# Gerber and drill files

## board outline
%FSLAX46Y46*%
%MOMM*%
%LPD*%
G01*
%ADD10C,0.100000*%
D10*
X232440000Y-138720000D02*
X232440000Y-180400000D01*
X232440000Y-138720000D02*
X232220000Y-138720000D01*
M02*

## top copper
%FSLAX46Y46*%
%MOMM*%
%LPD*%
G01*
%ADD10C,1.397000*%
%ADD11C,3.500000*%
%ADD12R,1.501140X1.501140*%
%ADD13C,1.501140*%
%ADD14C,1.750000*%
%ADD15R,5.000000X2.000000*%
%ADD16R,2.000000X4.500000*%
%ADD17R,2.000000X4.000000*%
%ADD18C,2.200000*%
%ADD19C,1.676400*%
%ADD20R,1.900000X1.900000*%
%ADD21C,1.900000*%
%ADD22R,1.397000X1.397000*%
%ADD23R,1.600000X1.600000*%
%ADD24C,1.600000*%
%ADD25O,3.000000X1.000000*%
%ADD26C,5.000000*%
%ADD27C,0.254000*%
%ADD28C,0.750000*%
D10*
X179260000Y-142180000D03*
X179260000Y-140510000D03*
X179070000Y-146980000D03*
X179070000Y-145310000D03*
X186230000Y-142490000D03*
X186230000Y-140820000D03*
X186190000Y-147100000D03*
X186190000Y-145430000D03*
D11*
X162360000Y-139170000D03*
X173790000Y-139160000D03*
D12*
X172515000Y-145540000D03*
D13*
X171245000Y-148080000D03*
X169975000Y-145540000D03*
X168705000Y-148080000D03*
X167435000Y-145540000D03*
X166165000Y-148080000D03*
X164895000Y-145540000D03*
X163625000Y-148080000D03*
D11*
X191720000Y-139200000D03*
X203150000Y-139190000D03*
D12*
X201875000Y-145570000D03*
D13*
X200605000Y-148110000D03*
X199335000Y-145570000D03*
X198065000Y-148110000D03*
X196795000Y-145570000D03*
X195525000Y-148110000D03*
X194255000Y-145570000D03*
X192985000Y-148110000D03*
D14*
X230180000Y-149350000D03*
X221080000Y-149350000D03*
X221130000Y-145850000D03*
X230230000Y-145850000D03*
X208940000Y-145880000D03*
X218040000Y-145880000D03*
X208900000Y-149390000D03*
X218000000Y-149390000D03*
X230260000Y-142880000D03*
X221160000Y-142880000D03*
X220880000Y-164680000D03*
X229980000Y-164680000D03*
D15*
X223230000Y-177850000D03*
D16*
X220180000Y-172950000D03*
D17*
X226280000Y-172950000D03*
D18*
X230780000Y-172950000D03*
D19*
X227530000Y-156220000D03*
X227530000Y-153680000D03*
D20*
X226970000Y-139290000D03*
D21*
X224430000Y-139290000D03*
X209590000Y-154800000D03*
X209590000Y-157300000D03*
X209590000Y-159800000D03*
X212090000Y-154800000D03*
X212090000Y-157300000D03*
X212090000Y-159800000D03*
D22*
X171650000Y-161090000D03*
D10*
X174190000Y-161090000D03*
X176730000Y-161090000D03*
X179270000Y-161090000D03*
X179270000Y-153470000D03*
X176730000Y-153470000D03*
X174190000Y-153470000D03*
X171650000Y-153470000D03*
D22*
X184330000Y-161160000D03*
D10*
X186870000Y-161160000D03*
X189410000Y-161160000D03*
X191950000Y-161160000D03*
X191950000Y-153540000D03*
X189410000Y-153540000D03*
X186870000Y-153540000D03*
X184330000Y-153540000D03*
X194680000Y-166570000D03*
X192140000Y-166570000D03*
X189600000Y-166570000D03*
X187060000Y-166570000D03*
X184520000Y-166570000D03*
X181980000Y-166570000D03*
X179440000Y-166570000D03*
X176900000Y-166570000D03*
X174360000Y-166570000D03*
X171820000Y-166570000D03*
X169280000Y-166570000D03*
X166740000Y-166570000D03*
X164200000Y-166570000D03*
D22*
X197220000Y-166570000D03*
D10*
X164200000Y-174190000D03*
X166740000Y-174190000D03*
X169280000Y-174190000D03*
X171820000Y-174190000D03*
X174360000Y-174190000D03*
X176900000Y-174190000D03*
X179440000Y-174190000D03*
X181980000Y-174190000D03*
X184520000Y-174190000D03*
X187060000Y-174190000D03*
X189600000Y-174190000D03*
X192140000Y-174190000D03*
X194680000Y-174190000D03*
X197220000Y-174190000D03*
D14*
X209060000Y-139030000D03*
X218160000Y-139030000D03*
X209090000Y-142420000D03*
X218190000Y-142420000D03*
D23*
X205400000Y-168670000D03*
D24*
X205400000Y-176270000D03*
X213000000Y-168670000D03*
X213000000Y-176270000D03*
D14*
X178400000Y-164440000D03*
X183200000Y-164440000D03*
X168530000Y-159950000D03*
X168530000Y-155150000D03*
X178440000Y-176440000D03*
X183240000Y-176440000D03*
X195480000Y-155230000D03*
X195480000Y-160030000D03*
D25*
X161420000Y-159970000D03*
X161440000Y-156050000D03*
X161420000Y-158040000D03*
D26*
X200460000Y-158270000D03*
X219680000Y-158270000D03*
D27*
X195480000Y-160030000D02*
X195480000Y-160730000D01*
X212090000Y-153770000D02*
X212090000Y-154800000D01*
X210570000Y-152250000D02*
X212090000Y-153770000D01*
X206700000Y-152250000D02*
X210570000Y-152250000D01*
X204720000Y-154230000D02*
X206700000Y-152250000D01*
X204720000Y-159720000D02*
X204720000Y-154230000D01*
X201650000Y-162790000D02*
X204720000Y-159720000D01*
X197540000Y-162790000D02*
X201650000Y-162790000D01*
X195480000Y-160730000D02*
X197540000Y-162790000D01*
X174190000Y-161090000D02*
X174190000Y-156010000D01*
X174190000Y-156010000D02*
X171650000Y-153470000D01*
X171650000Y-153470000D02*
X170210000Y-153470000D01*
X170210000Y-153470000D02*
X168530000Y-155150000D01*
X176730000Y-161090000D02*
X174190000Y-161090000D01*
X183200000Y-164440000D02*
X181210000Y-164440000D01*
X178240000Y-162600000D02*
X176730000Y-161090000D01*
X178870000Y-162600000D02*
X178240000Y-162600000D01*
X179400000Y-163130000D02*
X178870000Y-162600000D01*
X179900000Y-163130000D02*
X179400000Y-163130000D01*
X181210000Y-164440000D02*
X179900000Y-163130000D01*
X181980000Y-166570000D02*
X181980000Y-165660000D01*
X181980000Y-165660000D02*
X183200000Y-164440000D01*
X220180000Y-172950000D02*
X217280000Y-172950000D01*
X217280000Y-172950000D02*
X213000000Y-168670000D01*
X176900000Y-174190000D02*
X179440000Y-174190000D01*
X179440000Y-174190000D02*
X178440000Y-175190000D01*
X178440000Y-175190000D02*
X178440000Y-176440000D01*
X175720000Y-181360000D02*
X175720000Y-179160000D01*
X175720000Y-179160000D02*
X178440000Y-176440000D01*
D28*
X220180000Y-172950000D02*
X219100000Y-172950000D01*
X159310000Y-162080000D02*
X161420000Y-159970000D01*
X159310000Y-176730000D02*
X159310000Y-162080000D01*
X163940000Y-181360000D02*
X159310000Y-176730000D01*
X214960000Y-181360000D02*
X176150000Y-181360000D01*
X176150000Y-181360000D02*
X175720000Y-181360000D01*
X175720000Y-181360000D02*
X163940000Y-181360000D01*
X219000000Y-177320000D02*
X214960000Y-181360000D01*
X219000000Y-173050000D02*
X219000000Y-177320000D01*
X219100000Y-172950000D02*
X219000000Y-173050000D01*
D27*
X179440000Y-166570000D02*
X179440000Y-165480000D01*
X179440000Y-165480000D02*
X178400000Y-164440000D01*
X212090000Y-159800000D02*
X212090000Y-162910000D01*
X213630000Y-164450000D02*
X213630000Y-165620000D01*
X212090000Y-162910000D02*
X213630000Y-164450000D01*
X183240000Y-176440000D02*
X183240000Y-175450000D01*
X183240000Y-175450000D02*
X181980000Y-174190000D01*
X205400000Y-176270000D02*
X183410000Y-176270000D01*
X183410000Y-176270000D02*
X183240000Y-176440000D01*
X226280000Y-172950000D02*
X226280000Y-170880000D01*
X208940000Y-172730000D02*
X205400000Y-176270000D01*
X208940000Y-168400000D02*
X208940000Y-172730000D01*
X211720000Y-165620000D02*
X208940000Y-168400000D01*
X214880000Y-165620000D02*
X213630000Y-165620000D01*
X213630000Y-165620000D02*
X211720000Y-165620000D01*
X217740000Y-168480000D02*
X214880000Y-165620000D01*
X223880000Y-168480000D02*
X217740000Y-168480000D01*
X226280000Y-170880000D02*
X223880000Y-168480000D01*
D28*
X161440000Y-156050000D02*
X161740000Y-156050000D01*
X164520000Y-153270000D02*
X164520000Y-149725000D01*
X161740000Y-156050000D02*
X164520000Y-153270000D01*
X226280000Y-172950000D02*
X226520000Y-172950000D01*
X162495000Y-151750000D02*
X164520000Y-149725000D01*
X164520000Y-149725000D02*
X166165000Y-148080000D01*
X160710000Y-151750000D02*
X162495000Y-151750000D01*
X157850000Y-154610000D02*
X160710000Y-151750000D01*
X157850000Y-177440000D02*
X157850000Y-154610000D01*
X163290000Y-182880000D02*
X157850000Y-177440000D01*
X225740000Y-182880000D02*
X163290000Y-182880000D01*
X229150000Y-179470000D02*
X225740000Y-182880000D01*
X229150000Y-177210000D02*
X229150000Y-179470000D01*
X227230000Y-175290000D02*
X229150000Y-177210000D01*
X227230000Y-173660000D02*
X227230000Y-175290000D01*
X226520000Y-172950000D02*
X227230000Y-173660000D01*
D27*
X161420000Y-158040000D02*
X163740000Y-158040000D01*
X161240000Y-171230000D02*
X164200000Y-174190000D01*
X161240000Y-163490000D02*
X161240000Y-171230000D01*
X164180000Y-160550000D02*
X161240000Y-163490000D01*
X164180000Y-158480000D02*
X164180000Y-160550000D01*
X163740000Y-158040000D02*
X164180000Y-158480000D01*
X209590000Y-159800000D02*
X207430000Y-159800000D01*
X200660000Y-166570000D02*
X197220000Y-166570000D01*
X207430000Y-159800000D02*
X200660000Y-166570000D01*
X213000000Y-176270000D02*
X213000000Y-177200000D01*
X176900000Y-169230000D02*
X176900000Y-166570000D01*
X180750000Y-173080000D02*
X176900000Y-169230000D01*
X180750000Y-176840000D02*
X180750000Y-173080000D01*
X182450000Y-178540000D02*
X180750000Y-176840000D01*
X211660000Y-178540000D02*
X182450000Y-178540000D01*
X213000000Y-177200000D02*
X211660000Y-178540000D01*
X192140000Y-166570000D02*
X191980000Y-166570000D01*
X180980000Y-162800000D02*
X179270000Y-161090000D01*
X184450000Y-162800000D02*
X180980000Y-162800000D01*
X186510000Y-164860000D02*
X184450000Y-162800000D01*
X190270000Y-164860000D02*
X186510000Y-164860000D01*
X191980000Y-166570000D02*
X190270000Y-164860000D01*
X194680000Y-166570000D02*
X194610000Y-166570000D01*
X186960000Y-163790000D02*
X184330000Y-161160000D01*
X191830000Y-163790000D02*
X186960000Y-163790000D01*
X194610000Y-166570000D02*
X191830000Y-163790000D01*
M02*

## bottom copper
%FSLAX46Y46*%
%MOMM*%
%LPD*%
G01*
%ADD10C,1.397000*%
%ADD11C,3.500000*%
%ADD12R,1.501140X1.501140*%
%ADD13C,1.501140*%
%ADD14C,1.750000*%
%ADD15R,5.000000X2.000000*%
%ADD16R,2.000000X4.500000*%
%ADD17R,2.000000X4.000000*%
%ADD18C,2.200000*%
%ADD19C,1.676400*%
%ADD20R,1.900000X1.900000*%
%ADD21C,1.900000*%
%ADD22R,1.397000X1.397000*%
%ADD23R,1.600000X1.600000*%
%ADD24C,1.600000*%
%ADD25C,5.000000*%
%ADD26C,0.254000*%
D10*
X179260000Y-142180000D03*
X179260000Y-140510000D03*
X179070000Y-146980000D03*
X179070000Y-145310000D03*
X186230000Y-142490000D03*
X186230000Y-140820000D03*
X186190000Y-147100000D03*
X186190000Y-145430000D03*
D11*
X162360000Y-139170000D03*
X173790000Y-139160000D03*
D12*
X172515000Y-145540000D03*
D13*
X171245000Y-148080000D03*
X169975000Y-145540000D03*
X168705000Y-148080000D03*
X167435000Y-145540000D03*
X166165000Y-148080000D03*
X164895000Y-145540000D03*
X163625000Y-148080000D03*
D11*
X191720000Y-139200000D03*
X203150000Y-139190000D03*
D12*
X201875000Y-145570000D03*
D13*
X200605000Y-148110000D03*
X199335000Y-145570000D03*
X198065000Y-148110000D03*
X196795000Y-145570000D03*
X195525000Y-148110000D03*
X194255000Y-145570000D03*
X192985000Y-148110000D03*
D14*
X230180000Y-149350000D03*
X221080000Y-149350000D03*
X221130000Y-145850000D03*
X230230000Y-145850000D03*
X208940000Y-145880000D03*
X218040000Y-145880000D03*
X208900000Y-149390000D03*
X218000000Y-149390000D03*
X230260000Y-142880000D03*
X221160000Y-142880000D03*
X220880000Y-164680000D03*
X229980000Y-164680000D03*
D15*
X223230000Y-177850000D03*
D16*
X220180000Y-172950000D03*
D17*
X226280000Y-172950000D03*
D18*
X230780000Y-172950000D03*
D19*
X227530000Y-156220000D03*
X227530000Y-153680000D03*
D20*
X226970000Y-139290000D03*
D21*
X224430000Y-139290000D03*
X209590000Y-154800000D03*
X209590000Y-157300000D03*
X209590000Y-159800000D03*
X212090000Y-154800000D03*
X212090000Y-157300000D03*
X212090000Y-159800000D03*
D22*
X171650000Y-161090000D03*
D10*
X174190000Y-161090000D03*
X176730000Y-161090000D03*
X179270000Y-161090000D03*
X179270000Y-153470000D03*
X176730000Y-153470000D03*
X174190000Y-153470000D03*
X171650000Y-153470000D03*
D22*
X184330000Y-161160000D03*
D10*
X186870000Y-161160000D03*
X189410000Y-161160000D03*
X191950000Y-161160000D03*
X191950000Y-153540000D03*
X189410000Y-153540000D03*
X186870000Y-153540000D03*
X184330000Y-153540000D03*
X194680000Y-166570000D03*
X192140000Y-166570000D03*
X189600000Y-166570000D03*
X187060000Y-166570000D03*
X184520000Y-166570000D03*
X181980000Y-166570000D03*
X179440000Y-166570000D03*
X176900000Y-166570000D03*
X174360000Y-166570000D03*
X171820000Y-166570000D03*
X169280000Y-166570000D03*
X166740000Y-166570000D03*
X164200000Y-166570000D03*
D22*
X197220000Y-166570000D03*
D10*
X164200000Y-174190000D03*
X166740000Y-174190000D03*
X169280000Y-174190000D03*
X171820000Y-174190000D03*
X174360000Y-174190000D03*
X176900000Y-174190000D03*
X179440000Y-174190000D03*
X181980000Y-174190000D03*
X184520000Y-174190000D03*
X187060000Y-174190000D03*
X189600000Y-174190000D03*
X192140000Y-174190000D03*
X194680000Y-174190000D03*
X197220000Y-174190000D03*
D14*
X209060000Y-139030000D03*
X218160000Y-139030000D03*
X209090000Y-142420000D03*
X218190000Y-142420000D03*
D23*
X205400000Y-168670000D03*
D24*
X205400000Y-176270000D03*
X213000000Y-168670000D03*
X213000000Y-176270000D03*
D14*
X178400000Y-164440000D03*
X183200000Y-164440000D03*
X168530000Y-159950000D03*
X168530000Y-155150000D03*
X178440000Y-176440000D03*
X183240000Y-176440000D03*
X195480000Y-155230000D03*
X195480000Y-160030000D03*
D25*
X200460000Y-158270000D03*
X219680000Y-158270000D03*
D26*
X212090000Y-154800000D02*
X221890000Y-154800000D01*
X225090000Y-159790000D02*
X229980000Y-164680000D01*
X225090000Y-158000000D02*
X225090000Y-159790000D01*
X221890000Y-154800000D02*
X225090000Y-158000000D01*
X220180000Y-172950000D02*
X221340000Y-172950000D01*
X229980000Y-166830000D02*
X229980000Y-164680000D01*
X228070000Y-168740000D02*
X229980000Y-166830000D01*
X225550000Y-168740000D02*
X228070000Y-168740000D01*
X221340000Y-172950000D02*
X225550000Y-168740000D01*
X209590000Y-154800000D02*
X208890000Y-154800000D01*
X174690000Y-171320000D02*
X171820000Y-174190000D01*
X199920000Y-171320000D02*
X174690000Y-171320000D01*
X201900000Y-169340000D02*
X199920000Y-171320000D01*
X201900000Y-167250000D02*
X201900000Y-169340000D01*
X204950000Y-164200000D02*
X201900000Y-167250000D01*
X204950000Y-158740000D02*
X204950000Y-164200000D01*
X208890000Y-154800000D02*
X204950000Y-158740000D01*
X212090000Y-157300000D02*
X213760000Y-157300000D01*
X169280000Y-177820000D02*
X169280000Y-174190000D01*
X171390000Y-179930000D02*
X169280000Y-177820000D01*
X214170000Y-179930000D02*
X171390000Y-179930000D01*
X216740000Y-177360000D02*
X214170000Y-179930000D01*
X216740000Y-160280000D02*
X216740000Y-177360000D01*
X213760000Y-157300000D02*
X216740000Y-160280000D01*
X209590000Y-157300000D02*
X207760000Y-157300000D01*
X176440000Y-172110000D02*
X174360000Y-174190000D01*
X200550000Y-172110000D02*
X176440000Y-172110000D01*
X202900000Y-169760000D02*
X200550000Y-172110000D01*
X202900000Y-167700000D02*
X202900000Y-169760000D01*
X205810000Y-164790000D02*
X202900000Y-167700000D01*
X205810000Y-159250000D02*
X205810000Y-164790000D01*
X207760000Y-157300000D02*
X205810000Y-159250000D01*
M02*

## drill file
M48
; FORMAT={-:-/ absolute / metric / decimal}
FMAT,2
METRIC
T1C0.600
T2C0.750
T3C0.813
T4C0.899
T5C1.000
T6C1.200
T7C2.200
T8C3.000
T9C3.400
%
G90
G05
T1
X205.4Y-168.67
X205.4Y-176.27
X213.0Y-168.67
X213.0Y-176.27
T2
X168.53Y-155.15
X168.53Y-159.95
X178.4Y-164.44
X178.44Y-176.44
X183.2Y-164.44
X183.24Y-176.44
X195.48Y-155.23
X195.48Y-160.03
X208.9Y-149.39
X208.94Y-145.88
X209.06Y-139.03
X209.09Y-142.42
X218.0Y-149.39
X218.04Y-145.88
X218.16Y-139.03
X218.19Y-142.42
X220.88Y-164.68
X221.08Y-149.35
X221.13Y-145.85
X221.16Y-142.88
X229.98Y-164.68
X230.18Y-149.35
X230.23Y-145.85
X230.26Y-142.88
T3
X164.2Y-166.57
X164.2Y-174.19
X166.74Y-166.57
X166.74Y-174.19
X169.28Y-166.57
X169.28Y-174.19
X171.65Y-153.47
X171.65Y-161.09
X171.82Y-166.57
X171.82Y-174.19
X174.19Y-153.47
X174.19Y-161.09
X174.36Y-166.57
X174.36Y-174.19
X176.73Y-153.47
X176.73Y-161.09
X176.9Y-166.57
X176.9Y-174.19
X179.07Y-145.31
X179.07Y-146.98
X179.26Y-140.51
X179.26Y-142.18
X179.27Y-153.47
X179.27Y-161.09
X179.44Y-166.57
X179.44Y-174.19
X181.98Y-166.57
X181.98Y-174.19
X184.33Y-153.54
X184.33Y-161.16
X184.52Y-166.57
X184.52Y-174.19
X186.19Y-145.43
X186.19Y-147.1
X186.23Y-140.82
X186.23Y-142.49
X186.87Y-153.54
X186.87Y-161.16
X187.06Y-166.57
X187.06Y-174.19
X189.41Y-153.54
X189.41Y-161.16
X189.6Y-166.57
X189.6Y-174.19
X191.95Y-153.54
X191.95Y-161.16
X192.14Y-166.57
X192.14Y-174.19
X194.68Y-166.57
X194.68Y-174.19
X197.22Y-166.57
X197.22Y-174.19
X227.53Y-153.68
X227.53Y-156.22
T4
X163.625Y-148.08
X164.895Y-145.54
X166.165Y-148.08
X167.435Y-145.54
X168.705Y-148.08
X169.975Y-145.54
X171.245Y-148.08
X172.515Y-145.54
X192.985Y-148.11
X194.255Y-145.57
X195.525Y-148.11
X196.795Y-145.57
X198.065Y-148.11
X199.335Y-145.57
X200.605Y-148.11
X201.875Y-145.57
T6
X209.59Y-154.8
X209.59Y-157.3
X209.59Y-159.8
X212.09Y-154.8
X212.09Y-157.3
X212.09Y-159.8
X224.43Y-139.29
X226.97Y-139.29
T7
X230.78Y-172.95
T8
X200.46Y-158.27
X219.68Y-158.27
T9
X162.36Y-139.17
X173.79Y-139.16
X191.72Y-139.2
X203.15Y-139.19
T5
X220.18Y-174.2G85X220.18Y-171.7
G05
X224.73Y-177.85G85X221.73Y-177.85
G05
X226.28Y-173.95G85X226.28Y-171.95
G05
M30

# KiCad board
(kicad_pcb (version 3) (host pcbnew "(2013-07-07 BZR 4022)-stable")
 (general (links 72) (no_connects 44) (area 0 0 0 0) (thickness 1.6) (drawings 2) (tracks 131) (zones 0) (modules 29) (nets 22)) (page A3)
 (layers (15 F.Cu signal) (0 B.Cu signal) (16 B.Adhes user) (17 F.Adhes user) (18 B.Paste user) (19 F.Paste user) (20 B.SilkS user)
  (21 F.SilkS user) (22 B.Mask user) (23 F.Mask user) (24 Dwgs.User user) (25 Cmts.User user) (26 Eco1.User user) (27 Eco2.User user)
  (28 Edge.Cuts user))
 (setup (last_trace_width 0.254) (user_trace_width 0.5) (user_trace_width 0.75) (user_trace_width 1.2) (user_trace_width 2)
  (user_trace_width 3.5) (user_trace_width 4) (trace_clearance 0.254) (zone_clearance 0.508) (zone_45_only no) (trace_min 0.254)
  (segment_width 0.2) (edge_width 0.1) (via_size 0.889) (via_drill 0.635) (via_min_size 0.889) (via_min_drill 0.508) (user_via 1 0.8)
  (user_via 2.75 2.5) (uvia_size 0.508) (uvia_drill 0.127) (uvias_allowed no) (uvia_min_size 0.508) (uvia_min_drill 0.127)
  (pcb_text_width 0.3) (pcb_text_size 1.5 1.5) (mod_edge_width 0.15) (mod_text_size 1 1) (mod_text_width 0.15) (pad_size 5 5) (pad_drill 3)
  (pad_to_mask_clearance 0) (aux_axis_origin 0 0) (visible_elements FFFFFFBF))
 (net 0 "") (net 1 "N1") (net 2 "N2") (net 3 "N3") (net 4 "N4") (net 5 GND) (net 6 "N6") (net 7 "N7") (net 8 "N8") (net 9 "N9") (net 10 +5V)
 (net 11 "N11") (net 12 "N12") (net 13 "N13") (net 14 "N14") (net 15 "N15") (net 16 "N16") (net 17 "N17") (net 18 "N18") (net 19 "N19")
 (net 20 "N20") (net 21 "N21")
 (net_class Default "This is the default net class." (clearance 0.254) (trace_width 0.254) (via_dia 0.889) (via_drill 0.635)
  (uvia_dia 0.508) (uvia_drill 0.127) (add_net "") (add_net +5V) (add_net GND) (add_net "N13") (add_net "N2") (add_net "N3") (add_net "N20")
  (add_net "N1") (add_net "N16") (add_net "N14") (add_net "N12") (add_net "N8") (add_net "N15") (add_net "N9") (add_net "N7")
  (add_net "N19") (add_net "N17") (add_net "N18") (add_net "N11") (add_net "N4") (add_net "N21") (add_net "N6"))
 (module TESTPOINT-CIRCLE (layer F.Cu) (at 179.26 141.35 90)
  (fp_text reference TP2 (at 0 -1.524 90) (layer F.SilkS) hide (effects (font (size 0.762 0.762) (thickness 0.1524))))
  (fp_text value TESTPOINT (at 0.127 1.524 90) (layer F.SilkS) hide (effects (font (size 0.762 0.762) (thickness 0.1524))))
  (pad 1 thru_hole circle (at -0.83 0 90) (size 1.397 1.397) (drill 0.8128) (layers *.Cu *.Mask F.SilkS) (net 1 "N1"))
  (pad 1 thru_hole circle (at 0.84 0 90) (size 1.397 1.397) (drill 0.8128) (layers *.Cu *.Mask F.SilkS) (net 1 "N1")))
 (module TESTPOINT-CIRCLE (layer F.Cu) (at 179.07 146.15 90)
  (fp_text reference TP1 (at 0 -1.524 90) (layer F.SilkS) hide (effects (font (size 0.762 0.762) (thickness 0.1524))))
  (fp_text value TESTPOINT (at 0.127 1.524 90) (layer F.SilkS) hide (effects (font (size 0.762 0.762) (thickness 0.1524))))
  (pad 1 thru_hole circle (at -0.83 0 90) (size 1.397 1.397) (drill 0.8128) (layers *.Cu *.Mask F.SilkS) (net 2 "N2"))
  (pad 1 thru_hole circle (at 0.84 0 90) (size 1.397 1.397) (drill 0.8128) (layers *.Cu *.Mask F.SilkS) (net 2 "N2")))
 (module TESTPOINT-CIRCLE (layer F.Cu) (at 186.23 141.66 90)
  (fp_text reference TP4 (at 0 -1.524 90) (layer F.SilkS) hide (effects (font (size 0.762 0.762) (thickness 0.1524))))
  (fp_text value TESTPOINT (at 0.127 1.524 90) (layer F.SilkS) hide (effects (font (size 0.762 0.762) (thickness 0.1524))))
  (pad 1 thru_hole circle (at -0.83 0 90) (size 1.397 1.397) (drill 0.8128) (layers *.Cu *.Mask F.SilkS) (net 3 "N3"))
  (pad 1 thru_hole circle (at 0.84 0 90) (size 1.397 1.397) (drill 0.8128) (layers *.Cu *.Mask F.SilkS) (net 3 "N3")))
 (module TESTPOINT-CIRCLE (layer F.Cu) (at 186.19 146.27 90)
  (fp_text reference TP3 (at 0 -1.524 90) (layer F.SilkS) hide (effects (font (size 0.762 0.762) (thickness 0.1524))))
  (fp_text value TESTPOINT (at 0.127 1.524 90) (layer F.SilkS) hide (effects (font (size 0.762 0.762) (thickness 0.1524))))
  (pad 1 thru_hole circle (at -0.83 0 90) (size 1.397 1.397) (drill 0.8128) (layers *.Cu *.Mask F.SilkS) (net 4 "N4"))
  (pad 1 thru_hole circle (at 0.84 0 90) (size 1.397 1.397) (drill 0.8128) (layers *.Cu *.Mask F.SilkS) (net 4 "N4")))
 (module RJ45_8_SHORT (layer F.Cu) (at 168.07 139.19 180)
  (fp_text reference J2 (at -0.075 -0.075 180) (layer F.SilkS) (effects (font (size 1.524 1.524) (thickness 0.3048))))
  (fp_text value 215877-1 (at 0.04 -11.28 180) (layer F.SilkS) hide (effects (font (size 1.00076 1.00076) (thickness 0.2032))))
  (pad Hole thru_hole circle (at 5.71 0.02 180) (size 3.5 3.5) (drill 3.4) (layers *.Cu *.Mask F.SilkS))
  (pad Hole thru_hole circle (at -5.72 0.03 180) (size 3.5 3.5) (drill 3.4) (layers *.Cu *.Mask F.SilkS))
  (pad 1 thru_hole rect (at -4.445 -6.35 180) (size 1.50114 1.50114) (drill 0.89916) (layers *.Cu *.Mask F.SilkS) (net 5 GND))
  (pad 2 thru_hole circle (at -3.175 -8.89 180) (size 1.50114 1.50114) (drill 0.89916) (layers *.Cu *.Mask F.SilkS) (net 5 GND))
  (pad 3 thru_hole circle (at -1.905 -6.35 180) (size 1.50114 1.50114) (drill 0.89916) (layers *.Cu *.Mask F.SilkS) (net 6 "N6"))
  (pad 4 thru_hole circle (at -0.635 -8.89 180) (size 1.50114 1.50114) (drill 0.89916) (layers *.Cu *.Mask F.SilkS) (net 1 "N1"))
  (pad 5 thru_hole circle (at 0.635 -6.35 180) (size 1.50114 1.50114) (drill 0.89916) (layers *.Cu *.Mask F.SilkS) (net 2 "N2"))
  (pad 6 thru_hole circle (at 1.905 -8.89 180) (size 1.50114 1.50114) (drill 0.89916) (layers *.Cu *.Mask F.SilkS) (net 5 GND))
  (pad 7 thru_hole circle (at 3.175 -6.35 180) (size 1.50114 1.50114) (drill 0.89916) (layers *.Cu *.Mask F.SilkS) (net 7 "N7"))
  (pad 8 thru_hole circle (at 4.445 -8.89 180) (size 1.50114 1.50114) (drill 0.89916) (layers *.Cu *.Mask F.SilkS) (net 7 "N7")))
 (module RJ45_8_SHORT (layer F.Cu) (at 197.43 139.22 180)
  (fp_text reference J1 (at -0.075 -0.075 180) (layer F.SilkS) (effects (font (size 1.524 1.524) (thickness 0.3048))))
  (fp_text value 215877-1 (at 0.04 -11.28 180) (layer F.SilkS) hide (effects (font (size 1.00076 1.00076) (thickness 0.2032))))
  (pad Hole thru_hole circle (at 5.71 0.02 180) (size 3.5 3.5) (drill 3.4) (layers *.Cu *.Mask F.SilkS))
  (pad Hole thru_hole circle (at -5.72 0.03 180) (size 3.5 3.5) (drill 3.4) (layers *.Cu *.Mask F.SilkS))
  (pad 1 thru_hole rect (at -4.445 -6.35 180) (size 1.50114 1.50114) (drill 0.89916) (layers *.Cu *.Mask F.SilkS) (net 5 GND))
  (pad 2 thru_hole circle (at -3.175 -8.89 180) (size 1.50114 1.50114) (drill 0.89916) (layers *.Cu *.Mask F.SilkS) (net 5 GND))
  (pad 3 thru_hole circle (at -1.905 -6.35 180) (size 1.50114 1.50114) (drill 0.89916) (layers *.Cu *.Mask F.SilkS) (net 6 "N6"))
  (pad 4 thru_hole circle (at -0.635 -8.89 180) (size 1.50114 1.50114) (drill 0.89916) (layers *.Cu *.Mask F.SilkS) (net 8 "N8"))
  (pad 5 thru_hole circle (at 0.635 -6.35 180) (size 1.50114 1.50114) (drill 0.89916) (layers *.Cu *.Mask F.SilkS) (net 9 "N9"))
  (pad 6 thru_hole circle (at 1.905 -8.89 180) (size 1.50114 1.50114) (drill 0.89916) (layers *.Cu *.Mask F.SilkS) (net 5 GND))
  (pad 7 thru_hole circle (at 3.175 -6.35 180) (size 1.50114 1.50114) (drill 0.89916) (layers *.Cu *.Mask F.SilkS) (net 7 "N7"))
  (pad 8 thru_hole circle (at 4.445 -8.89 180) (size 1.50114 1.50114) (drill 0.89916) (layers *.Cu *.Mask F.SilkS) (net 7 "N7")))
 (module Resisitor (layer F.Cu) (at 225.58 149.35 180)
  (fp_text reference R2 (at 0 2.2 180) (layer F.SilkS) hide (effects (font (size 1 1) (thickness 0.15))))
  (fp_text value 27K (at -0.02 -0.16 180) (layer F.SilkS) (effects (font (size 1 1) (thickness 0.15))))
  (pad 1 thru_hole circle (at -4.6 0 180) (size 1.75 1.75) (drill 0.75) (layers *.Cu *.Mask F.SilkS) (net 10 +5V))
  (pad 2 thru_hole circle (at 4.5 0 180) (size 1.75 1.75) (drill 0.75) (layers *.Cu *.Mask F.SilkS) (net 4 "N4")))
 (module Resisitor (layer F.Cu) (at 225.73 145.85)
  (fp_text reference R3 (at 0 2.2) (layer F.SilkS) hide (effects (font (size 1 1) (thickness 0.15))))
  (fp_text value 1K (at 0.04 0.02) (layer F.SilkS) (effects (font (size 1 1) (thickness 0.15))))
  (pad 1 thru_hole circle (at -4.6 0) (size 1.75 1.75) (drill 0.75) (layers *.Cu *.Mask F.SilkS) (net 4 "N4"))
  (pad 2 thru_hole circle (at 4.5 0) (size 1.75 1.75) (drill 0.75) (layers *.Cu *.Mask F.SilkS) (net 9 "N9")))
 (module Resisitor (layer F.Cu) (at 213.54 145.88)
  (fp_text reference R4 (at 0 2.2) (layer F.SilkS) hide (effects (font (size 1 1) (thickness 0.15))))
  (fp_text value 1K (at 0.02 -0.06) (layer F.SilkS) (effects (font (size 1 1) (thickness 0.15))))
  (pad 1 thru_hole circle (at -4.6 0) (size 1.75 1.75) (drill 0.75) (layers *.Cu *.Mask F.SilkS) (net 8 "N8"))
  (pad 2 thru_hole circle (at 4.5 0) (size 1.75 1.75) (drill 0.75) (layers *.Cu *.Mask F.SilkS) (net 3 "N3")))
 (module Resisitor (layer F.Cu) (at 213.5 149.39)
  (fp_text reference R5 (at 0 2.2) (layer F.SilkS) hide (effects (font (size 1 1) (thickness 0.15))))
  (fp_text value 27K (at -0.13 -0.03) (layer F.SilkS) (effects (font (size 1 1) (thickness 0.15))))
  (pad 1 thru_hole circle (at -4.6 0) (size 1.75 1.75) (drill 0.75) (layers *.Cu *.Mask F.SilkS) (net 3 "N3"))
  (pad 2 thru_hole circle (at 4.5 0) (size 1.75 1.75) (drill 0.75) (layers *.Cu *.Mask F.SilkS) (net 5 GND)))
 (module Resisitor (layer F.Cu) (at 225.66 142.88 180)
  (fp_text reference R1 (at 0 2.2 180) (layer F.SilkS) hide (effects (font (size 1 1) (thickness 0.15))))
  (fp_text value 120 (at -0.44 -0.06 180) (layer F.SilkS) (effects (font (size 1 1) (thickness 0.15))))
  (pad 1 thru_hole circle (at -4.6 0 180) (size 1.75 1.75) (drill 0.75) (layers *.Cu *.Mask F.SilkS) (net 9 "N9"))
  (pad 2 thru_hole circle (at 4.5 0 180) (size 1.75 1.75) (drill 0.75) (layers *.Cu *.Mask F.SilkS) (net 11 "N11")))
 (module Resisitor (layer F.Cu) (at 225.48 164.68)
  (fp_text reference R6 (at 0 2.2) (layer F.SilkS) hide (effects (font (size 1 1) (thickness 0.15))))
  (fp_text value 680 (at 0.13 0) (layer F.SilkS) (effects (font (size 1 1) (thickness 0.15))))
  (pad 1 thru_hole circle (at -4.6 0) (size 1.75 1.75) (drill 0.75) (layers *.Cu *.Mask F.SilkS) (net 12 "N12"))
  (pad 2 thru_hole circle (at 4.5 0) (size 1.75 1.75) (drill 0.75) (layers *.Cu *.Mask F.SilkS) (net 10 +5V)))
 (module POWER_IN (layer F.Cu) (at 227.38 176.02 180)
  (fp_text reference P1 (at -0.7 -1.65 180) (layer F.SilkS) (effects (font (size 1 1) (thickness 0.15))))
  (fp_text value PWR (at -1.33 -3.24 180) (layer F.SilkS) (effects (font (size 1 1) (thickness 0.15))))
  (pad "" thru_hole rect (at 4.15 -1.83 180) (size 5 2) (drill oval 4 1) (layers *.Cu *.Mask F.SilkS))
  (pad 1 thru_hole rect (at 7.2 3.07 180) (size 2 4.5) (drill oval 1 3.5) (layers *.Cu *.Mask F.SilkS) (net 10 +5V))
  (pad 2 thru_hole rect (at 1.1 3.07 180) (size 2 4) (drill oval 1 3) (layers *.Cu *.Mask F.SilkS) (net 5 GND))
  (pad "" thru_hole circle (at -3.4 3.07 180) (size 2.2 2.2) (drill 2.2) (layers *.Cu *.Mask F.SilkS)))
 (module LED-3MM (layer F.Cu) (at 227.53 154.95 90)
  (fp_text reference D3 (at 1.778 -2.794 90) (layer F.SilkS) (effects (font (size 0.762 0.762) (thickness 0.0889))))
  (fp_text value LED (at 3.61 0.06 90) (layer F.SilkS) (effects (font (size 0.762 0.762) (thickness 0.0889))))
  (pad 1 thru_hole circle (at -1.27 0 90) (size 1.6764 1.6764) (drill 0.8128) (layers *.Cu *.Mask F.SilkS) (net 12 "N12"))
  (pad 2 thru_hole circle (at 1.27 0 90) (size 1.6764 1.6764) (drill 0.8128) (layers *.Cu *.Mask F.SilkS) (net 5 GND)))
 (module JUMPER (layer F.Cu) (at 225.7 139.29 180)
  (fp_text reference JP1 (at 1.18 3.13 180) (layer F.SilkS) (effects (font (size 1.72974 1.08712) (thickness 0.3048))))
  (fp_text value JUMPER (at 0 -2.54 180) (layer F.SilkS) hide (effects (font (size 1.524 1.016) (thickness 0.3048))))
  (pad 1 thru_hole rect (at -1.27 0 180) (size 1.9 1.9) (drill 1.2) (layers *.Cu *.Mask F.SilkS) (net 11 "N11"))
  (pad 2 thru_hole circle (at 1.27 0 180) (size 1.9 1.9) (drill 1.2) (layers *.Cu *.Mask F.SilkS) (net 8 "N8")))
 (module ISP (layer F.Cu) (at 210.69 157.8 90)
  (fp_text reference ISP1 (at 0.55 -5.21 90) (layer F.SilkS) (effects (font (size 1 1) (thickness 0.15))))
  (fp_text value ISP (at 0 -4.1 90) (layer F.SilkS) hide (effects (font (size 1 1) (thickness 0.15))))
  (pad 1 thru_hole circle (at 3 -1.1 90) (size 1.9 1.9) (drill 1.2) (layers *.Cu *.Mask F.SilkS) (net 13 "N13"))
  (pad 3 thru_hole circle (at 0.5 -1.1 90) (size 1.9 1.9) (drill 1.2) (layers *.Cu *.Mask F.SilkS) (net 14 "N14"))
  (pad 5 thru_hole circle (at -2 -1.1 90) (size 1.9 1.9) (drill 1.2) (layers *.Cu *.Mask F.SilkS) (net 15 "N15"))
  (pad 2 thru_hole circle (at 3 1.4 90) (size 1.9 1.9) (drill 1.2) (layers *.Cu *.Mask F.SilkS) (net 10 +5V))
  (pad 4 thru_hole circle (at 0.5 1.4 90) (size 1.9 1.9) (drill 1.2) (layers *.Cu *.Mask F.SilkS) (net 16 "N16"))
  (pad 6 thru_hole circle (at -2 1.4 90) (size 1.9 1.9) (drill 1.2) (layers *.Cu *.Mask F.SilkS) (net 5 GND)))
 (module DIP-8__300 (layer F.Cu) (at 175.46 157.28)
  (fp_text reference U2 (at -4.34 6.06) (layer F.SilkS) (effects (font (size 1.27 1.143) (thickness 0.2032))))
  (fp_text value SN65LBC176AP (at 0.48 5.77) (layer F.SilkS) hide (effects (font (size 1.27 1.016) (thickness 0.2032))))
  (pad 1 thru_hole rect (at -3.81 3.81) (size 1.397 1.397) (drill 0.8128) (layers *.Cu *.Mask F.SilkS))
  (pad 2 thru_hole circle (at -1.27 3.81) (size 1.397 1.397) (drill 0.8128) (layers *.Cu *.Mask F.SilkS) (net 10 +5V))
  (pad 3 thru_hole circle (at 1.27 3.81) (size 1.397 1.397) (drill 0.8128) (layers *.Cu *.Mask F.SilkS) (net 10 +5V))
  (pad 4 thru_hole circle (at 3.81 3.81) (size 1.397 1.397) (drill 0.8128) (layers *.Cu *.Mask F.SilkS) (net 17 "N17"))
  (pad 5 thru_hole circle (at 3.81 -3.81) (size 1.397 1.397) (drill 0.8128) (layers *.Cu *.Mask F.SilkS) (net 5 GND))
  (pad 6 thru_hole circle (at 1.27 -3.81) (size 1.397 1.397) (drill 0.8128) (layers *.Cu *.Mask F.SilkS) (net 2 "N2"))
  (pad 7 thru_hole circle (at -1.27 -3.81) (size 1.397 1.397) (drill 0.8128) (layers *.Cu *.Mask F.SilkS) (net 1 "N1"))
  (pad 8 thru_hole circle (at -3.81 -3.81) (size 1.397 1.397) (drill 0.8128) (layers *.Cu *.Mask F.SilkS) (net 10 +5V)))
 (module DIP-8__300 (layer F.Cu) (at 188.14 157.35)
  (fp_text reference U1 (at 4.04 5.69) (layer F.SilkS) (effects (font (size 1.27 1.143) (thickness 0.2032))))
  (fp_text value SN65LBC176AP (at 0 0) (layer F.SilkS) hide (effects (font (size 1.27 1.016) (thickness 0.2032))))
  (pad 1 thru_hole rect (at -3.81 3.81) (size 1.397 1.397) (drill 0.8128) (layers *.Cu *.Mask F.SilkS) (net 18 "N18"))
  (pad 2 thru_hole circle (at -1.27 3.81) (size 1.397 1.397) (drill 0.8128) (layers *.Cu *.Mask F.SilkS) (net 5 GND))
  (pad 3 thru_hole circle (at 1.27 3.81) (size 1.397 1.397) (drill 0.8128) (layers *.Cu *.Mask F.SilkS) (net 5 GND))
  (pad 4 thru_hole circle (at 3.81 3.81) (size 1.397 1.397) (drill 0.8128) (layers *.Cu *.Mask F.SilkS))
  (pad 5 thru_hole circle (at 3.81 -3.81) (size 1.397 1.397) (drill 0.8128) (layers *.Cu *.Mask F.SilkS) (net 5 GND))
  (pad 6 thru_hole circle (at 1.27 -3.81) (size 1.397 1.397) (drill 0.8128) (layers *.Cu *.Mask F.SilkS) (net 4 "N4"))
  (pad 7 thru_hole circle (at -1.27 -3.81) (size 1.397 1.397) (drill 0.8128) (layers *.Cu *.Mask F.SilkS) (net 3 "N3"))
  (pad 8 thru_hole circle (at -3.81 -3.81) (size 1.397 1.397) (drill 0.8128) (layers *.Cu *.Mask F.SilkS) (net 10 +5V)))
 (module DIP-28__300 (layer F.Cu) (at 180.71 170.38 180)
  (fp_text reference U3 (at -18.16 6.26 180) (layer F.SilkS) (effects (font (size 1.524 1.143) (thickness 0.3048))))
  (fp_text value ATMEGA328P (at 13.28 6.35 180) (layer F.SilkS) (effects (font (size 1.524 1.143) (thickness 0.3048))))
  (pad 2 thru_hole circle (at -13.97 3.81 180) (size 1.397 1.397) (drill 0.8128) (layers *.Cu *.Mask F.SilkS) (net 18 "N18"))
  (pad 3 thru_hole circle (at -11.43 3.81 180) (size 1.397 1.397) (drill 0.8128) (layers *.Cu *.Mask F.SilkS) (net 17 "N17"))
  (pad 4 thru_hole circle (at -8.89 3.81 180) (size 1.397 1.397) (drill 0.8128) (layers *.Cu *.Mask F.SilkS))
  (pad 5 thru_hole circle (at -6.35 3.81 180) (size 1.397 1.397) (drill 0.8128) (layers *.Cu *.Mask F.SilkS))
  (pad 6 thru_hole circle (at -3.81 3.81 180) (size 1.397 1.397) (drill 0.8128) (layers *.Cu *.Mask F.SilkS))
  (pad 7 thru_hole circle (at -1.27 3.81 180) (size 1.397 1.397) (drill 0.8128) (layers *.Cu *.Mask F.SilkS) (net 10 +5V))
  (pad 8 thru_hole circle (at 1.27 3.81 180) (size 1.397 1.397) (drill 0.8128) (layers *.Cu *.Mask F.SilkS) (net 5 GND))
  (pad 9 thru_hole circle (at 3.81 3.81 180) (size 1.397 1.397) (drill 0.8128) (layers *.Cu *.Mask F.SilkS) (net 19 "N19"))
  (pad 10 thru_hole circle (at 6.35 3.81 180) (size 1.397 1.397) (drill 0.8128) (layers *.Cu *.Mask F.SilkS))
  (pad 11 thru_hole circle (at 8.89 3.81 180) (size 1.397 1.397) (drill 0.8128) (layers *.Cu *.Mask F.SilkS))
  (pad 12 thru_hole circle (at 11.43 3.81 180) (size 1.397 1.397) (drill 0.8128) (layers *.Cu *.Mask F.SilkS))
  (pad 13 thru_hole circle (at 13.97 3.81 180) (size 1.397 1.397) (drill 0.8128) (layers *.Cu *.Mask F.SilkS))
  (pad 14 thru_hole circle (at 16.51 3.81 180) (size 1.397 1.397) (drill 0.8128) (layers *.Cu *.Mask F.SilkS))
  (pad 1 thru_hole rect (at -16.51 3.81 180) (size 1.397 1.397) (drill 0.8128) (layers *.Cu *.Mask F.SilkS) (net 15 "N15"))
  (pad 15 thru_hole circle (at 16.51 -3.81 180) (size 1.397 1.397) (drill 0.8128) (layers *.Cu *.Mask F.SilkS) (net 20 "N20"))
  (pad 16 thru_hole circle (at 13.97 -3.81 180) (size 1.397 1.397) (drill 0.8128) (layers *.Cu *.Mask F.SilkS))
  (pad 17 thru_hole circle (at 11.43 -3.81 180) (size 1.397 1.397) (drill 0.8128) (layers *.Cu *.Mask F.SilkS) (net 16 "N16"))
  (pad 18 thru_hole circle (at 8.89 -3.81 180) (size 1.397 1.397) (drill 0.8128) (layers *.Cu *.Mask F.SilkS) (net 13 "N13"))
  (pad 19 thru_hole circle (at 6.35 -3.81 180) (size 1.397 1.397) (drill 0.8128) (layers *.Cu *.Mask F.SilkS) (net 14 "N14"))
  (pad 20 thru_hole circle (at 3.81 -3.81 180) (size 1.397 1.397) (drill 0.8128) (layers *.Cu *.Mask F.SilkS) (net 10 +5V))
  (pad 21 thru_hole circle (at 1.27 -3.81 180) (size 1.397 1.397) (drill 0.8128) (layers *.Cu *.Mask F.SilkS) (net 10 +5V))
  (pad 22 thru_hole circle (at -1.27 -3.81 180) (size 1.397 1.397) (drill 0.8128) (layers *.Cu *.Mask F.SilkS) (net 5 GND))
  (pad 23 thru_hole circle (at -3.81 -3.81 180) (size 1.397 1.397) (drill 0.8128) (layers *.Cu *.Mask F.SilkS))
  (pad 24 thru_hole circle (at -6.35 -3.81 180) (size 1.397 1.397) (drill 0.8128) (layers *.Cu *.Mask F.SilkS))
  (pad 25 thru_hole circle (at -8.89 -3.81 180) (size 1.397 1.397) (drill 0.8128) (layers *.Cu *.Mask F.SilkS))
  (pad 26 thru_hole circle (at -11.43 -3.81 180) (size 1.397 1.397) (drill 0.8128) (layers *.Cu *.Mask F.SilkS))
  (pad 27 thru_hole circle (at -13.97 -3.81 180) (size 1.397 1.397) (drill 0.8128) (layers *.Cu *.Mask F.SilkS))
  (pad 28 thru_hole circle (at -16.51 -3.81 180) (size 1.397 1.397) (drill 0.8128) (layers *.Cu *.Mask F.SilkS)))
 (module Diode (layer F.Cu) (at 213.66 139.03)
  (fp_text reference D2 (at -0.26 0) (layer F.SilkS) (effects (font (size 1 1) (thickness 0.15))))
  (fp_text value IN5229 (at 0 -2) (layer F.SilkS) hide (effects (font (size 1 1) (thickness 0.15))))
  (pad 1 thru_hole circle (at -4.6 0) (size 1.75 1.75) (drill 0.75) (layers *.Cu *.Mask F.SilkS) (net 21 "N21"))
  (pad 2 thru_hole circle (at 4.5 0) (size 1.75 1.75) (drill 0.75) (layers *.Cu *.Mask F.SilkS) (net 5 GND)))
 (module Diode (layer F.Cu) (at 213.69 142.42)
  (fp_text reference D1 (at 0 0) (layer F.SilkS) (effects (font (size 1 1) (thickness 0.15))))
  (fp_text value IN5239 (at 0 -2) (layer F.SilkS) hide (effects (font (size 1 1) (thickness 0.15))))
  (pad 1 thru_hole circle (at -4.6 0) (size 1.75 1.75) (drill 0.75) (layers *.Cu *.Mask F.SilkS) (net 21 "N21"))
  (pad 2 thru_hole circle (at 4.5 0) (size 1.75 1.75) (drill 0.75) (layers *.Cu *.Mask F.SilkS) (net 3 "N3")))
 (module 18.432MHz (layer F.Cu) (at 209 172.02)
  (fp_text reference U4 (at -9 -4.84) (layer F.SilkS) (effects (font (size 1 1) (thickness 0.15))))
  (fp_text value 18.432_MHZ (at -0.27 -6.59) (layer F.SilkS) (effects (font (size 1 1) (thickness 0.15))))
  (pad 1 thru_hole rect (at -3.6 -3.35) (size 1.6 1.6) (drill 0.6) (layers *.Cu *.Mask F.SilkS))
  (pad 4 thru_hole circle (at -3.6 4.25) (size 1.6 1.6) (drill 0.6) (layers *.Cu *.Mask F.SilkS) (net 5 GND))
  (pad 8 thru_hole circle (at 4 -3.35) (size 1.6 1.6) (drill 0.6) (layers *.Cu *.Mask F.SilkS) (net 10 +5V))
  (pad 5 thru_hole circle (at 4 4.25) (size 1.6 1.6) (drill 0.6) (layers *.Cu *.Mask F.SilkS) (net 19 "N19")))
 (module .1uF (layer F.Cu) (at 180.9 164.44)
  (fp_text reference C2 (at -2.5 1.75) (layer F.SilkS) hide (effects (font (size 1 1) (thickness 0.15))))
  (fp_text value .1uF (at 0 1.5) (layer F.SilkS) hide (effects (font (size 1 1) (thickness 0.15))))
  (pad 1 thru_hole circle (at -2.5 0) (size 1.75 1.75) (drill 0.75) (layers *.Cu *.Mask F.SilkS) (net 5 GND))
  (pad 2 thru_hole circle (at 2.3 0) (size 1.75 1.75) (drill 0.75) (layers *.Cu *.Mask F.SilkS) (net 10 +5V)))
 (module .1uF (layer F.Cu) (at 168.53 157.45 90)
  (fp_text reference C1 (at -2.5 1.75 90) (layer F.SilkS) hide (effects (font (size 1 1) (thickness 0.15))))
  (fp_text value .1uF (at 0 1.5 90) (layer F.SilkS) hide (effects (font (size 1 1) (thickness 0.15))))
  (pad 1 thru_hole circle (at -2.5 0 90) (size 1.75 1.75) (drill 0.75) (layers *.Cu *.Mask F.SilkS) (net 5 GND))
  (pad 2 thru_hole circle (at 2.3 0 90) (size 1.75 1.75) (drill 0.75) (layers *.Cu *.Mask F.SilkS) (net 10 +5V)))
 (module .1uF (layer F.Cu) (at 180.94 176.44)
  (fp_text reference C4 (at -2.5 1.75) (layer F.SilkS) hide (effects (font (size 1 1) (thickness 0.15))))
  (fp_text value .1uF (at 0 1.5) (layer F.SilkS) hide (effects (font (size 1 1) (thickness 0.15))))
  (pad 1 thru_hole circle (at -2.5 0) (size 1.75 1.75) (drill 0.75) (layers *.Cu *.Mask F.SilkS) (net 10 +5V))
  (pad 2 thru_hole circle (at 2.3 0) (size 1.75 1.75) (drill 0.75) (layers *.Cu *.Mask F.SilkS) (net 5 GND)))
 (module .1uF (layer F.Cu) (at 195.48 157.73 270)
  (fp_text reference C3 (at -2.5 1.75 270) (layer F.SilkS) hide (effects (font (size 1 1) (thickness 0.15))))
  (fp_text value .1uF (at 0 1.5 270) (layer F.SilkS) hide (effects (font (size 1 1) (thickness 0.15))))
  (pad 1 thru_hole circle (at -2.5 0 270) (size 1.75 1.75) (drill 0.75) (layers *.Cu *.Mask F.SilkS) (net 5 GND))
  (pad 2 thru_hole circle (at 2.3 0 270) (size 1.75 1.75) (drill 0.75) (layers *.Cu *.Mask F.SilkS) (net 10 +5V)))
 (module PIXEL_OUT (layer F.Cu) (at 161.42 158.04 270)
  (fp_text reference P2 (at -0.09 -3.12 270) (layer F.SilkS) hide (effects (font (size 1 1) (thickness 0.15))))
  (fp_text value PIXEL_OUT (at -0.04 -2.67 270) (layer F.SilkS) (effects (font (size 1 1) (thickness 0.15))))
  (pad 1 smd oval (at 1.93 0 270) (size 1 3) (layers F.Cu F.Paste F.Mask) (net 10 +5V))
  (pad 2 smd oval (at -1.99 -0.02 270) (size 1 3) (layers F.Cu F.Paste F.Mask) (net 5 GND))
  (pad 3 smd oval (at 0 0 270) (size 1 3) (layers F.Cu F.Paste F.Mask) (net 20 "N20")))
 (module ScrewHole (layer F.Cu) (at 200.46 158.27)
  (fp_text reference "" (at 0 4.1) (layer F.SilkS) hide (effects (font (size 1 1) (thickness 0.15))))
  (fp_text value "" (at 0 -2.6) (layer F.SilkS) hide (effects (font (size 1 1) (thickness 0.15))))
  (pad "" thru_hole circle (at 0 0) (size 5 5) (drill 3) (layers *.Cu *.Mask F.SilkS)))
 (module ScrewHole (layer F.Cu) (at 219.68 158.27)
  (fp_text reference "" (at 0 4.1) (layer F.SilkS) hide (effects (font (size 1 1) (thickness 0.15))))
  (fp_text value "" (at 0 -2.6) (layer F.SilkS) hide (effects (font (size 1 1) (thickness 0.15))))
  (pad "" thru_hole circle (at 0 0) (size 5 5) (drill 3) (layers *.Cu *.Mask F.SilkS)))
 (gr_line (start 232.44 138.72) (end 232.44 180.4) (angle 90) (layer Edge.Cuts) (width 0.1))
 (gr_line (start 232.44 138.72) (end 232.22 138.72) (angle 90) (layer Edge.Cuts) (width 0.1))
 (segment (start 195.48 160.03) (end 195.48 160.73) (width 0.254) (layer F.Cu) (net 10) (status C00000))
 (segment (start 212.09 153.77) (end 212.09 154.8) (width 0.254) (layer F.Cu) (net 10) (status 800000))
 (segment (start 210.57 152.25) (end 212.09 153.77) (width 0.254) (layer F.Cu) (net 10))
 (segment (start 206.7 152.25) (end 210.57 152.25) (width 0.254) (layer F.Cu) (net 10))
 (segment (start 204.72 154.23) (end 206.7 152.25) (width 0.254) (layer F.Cu) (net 10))
 (segment (start 204.72 159.72) (end 204.72 154.23) (width 0.254) (layer F.Cu) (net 10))
 (segment (start 201.65 162.79) (end 204.72 159.72) (width 0.254) (layer F.Cu) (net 10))
 (segment (start 197.54 162.79) (end 201.65 162.79) (width 0.254) (layer F.Cu) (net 10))
 (segment (start 195.48 160.73) (end 197.54 162.79) (width 0.254) (layer F.Cu) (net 10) (status 400000))
 (segment (start 174.19 161.09) (end 174.19 156.01) (width 0.254) (layer F.Cu) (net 10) (status 400000))
 (segment (start 174.19 156.01) (end 171.65 153.47) (width 0.254) (layer F.Cu) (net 10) (status 800000))
 (segment (start 171.65 153.47) (end 170.21 153.47) (width 0.254) (layer F.Cu) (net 10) (status 400000))
 (segment (start 170.21 153.47) (end 168.53 155.15) (width 0.254) (layer F.Cu) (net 10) (status 800000))
 (segment (start 176.73 161.09) (end 174.19 161.09) (width 0.254) (layer F.Cu) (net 10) (status C00000))
 (segment (start 183.2 164.44) (end 181.21 164.44) (width 0.254) (layer F.Cu) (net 10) (status 400000))
 (segment (start 178.24 162.6) (end 176.73 161.09) (width 0.254) (layer F.Cu) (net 10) (status 800000))
 (segment (start 178.87 162.6) (end 178.24 162.6) (width 0.254) (layer F.Cu) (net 10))
 (segment (start 179.4 163.13) (end 178.87 162.6) (width 0.254) (layer F.Cu) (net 10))
 (segment (start 179.9 163.13) (end 179.4 163.13) (width 0.254) (layer F.Cu) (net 10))
 (segment (start 181.21 164.44) (end 179.9 163.13) (width 0.254) (layer F.Cu) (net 10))
 (segment (start 181.98 166.57) (end 181.98 165.66) (width 0.254) (layer F.Cu) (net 10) (status 400000))
 (segment (start 181.98 165.66) (end 183.2 164.44) (width 0.254) (layer F.Cu) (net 10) (status 800000))
 (segment (start 212.09 154.8) (end 221.89 154.8) (width 0.254) (layer B.Cu) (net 10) (status 400000))
 (segment (start 225.09 159.79) (end 229.98 164.68) (width 0.254) (layer B.Cu) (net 10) (status 800000))
 (segment (start 225.09 158) (end 225.09 159.79) (width 0.254) (layer B.Cu) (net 10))
 (segment (start 221.89 154.8) (end 225.09 158) (width 0.254) (layer B.Cu) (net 10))
 (segment (start 220.18 172.95) (end 221.34 172.95) (width 0.254) (layer B.Cu) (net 10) (status 400000))
 (segment (start 229.98 166.83) (end 229.98 164.68) (width 0.254) (layer B.Cu) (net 10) (status 800000))
 (segment (start 228.07 168.74) (end 229.98 166.83) (width 0.254) (layer B.Cu) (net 10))
 (segment (start 225.55 168.74) (end 228.07 168.74) (width 0.254) (layer B.Cu) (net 10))
 (segment (start 221.34 172.95) (end 225.55 168.74) (width 0.254) (layer B.Cu) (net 10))
 (segment (start 220.18 172.95) (end 217.28 172.95) (width 0.254) (layer F.Cu) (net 10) (status 400000))
 (segment (start 217.28 172.95) (end 213 168.67) (width 0.254) (layer F.Cu) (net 10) (status 800000))
 (segment (start 176.9 174.19) (end 179.44 174.19) (width 0.254) (layer F.Cu) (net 10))
 (segment (start 179.44 174.19) (end 178.44 175.19) (width 0.254) (layer F.Cu) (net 10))
 (segment (start 178.44 175.19) (end 178.44 176.44) (width 0.254) (layer F.Cu) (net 10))
 (segment (start 175.72 181.36) (end 175.72 179.16) (width 0.254) (layer F.Cu) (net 10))
 (segment (start 175.72 179.16) (end 178.44 176.44) (width 0.254) (layer F.Cu) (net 10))
 (segment (start 220.18 172.95) (end 219.1 172.95) (width 0.75) (layer F.Cu) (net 10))
 (segment (start 159.31 162.08) (end 161.42 159.97) (width 0.75) (layer F.Cu) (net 10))
 (segment (start 159.31 176.73) (end 159.31 162.08) (width 0.75) (layer F.Cu) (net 10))
 (segment (start 163.94 181.36) (end 159.31 176.73) (width 0.75) (layer F.Cu) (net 10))
 (segment (start 214.96 181.36) (end 176.15 181.36) (width 0.75) (layer F.Cu) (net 10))
 (segment (start 176.15 181.36) (end 175.72 181.36) (width 0.75) (layer F.Cu) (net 10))
 (segment (start 175.72 181.36) (end 163.94 181.36) (width 0.75) (layer F.Cu) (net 10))
 (segment (start 219 177.32) (end 214.96 181.36) (width 0.75) (layer F.Cu) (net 10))
 (segment (start 219 173.05) (end 219 177.32) (width 0.75) (layer F.Cu) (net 10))
 (segment (start 219.1 172.95) (end 219 173.05) (width 0.75) (layer F.Cu) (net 10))
 (segment (start 179.44 166.57) (end 179.44 165.48) (width 0.254) (layer F.Cu) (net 5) (status 400000))
 (segment (start 179.44 165.48) (end 178.4 164.44) (width 0.254) (layer F.Cu) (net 5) (status 800000))
 (segment (start 212.09 159.8) (end 212.09 162.91) (width 0.254) (layer F.Cu) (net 5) (status 400000))
 (segment (start 213.63 164.45) (end 213.63 165.62) (width 0.254) (layer F.Cu) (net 5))
 (segment (start 212.09 162.91) (end 213.63 164.45) (width 0.254) (layer F.Cu) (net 5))
 (segment (start 183.24 176.44) (end 183.24 175.45) (width 0.254) (layer F.Cu) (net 5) (status 400000))
 (segment (start 183.24 175.45) (end 181.98 174.19) (width 0.254) (layer F.Cu) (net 5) (status 800000))
 (segment (start 205.4 176.27) (end 183.41 176.27) (width 0.254) (layer F.Cu) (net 5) (status C00000))
 (segment (start 183.41 176.27) (end 183.24 176.44) (width 0.254) (layer F.Cu) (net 5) (status C00000))
 (segment (start 226.28 172.95) (end 226.28 170.88) (width 0.254) (layer F.Cu) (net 5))
 (segment (start 208.94 172.73) (end 205.4 176.27) (width 0.254) (layer F.Cu) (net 5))
 (segment (start 208.94 168.4) (end 208.94 172.73) (width 0.254) (layer F.Cu) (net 5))
 (segment (start 211.72 165.62) (end 208.94 168.4) (width 0.254) (layer F.Cu) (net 5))
 (segment (start 214.88 165.62) (end 213.63 165.62) (width 0.254) (layer F.Cu) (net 5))
 (segment (start 213.63 165.62) (end 211.72 165.62) (width 0.254) (layer F.Cu) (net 5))
 (segment (start 217.74 168.48) (end 214.88 165.62) (width 0.254) (layer F.Cu) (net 5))
 (segment (start 223.88 168.48) (end 217.74 168.48) (width 0.254) (layer F.Cu) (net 5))
 (segment (start 226.28 170.88) (end 223.88 168.48) (width 0.254) (layer F.Cu) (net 5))
 (segment (start 161.44 156.05) (end 161.74 156.05) (width 0.75) (layer F.Cu) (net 5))
 (segment (start 164.52 153.27) (end 164.52 149.725) (width 0.75) (layer F.Cu) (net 5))
 (segment (start 161.74 156.05) (end 164.52 153.27) (width 0.75) (layer F.Cu) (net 5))
 (segment (start 226.28 172.95) (end 226.52 172.95) (width 0.75) (layer F.Cu) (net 5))
 (segment (start 162.495 151.75) (end 164.52 149.725) (width 0.75) (layer F.Cu) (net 5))
 (segment (start 164.52 149.725) (end 166.165 148.08) (width 0.75) (layer F.Cu) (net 5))
 (segment (start 160.71 151.75) (end 162.495 151.75) (width 0.75) (layer F.Cu) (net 5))
 (segment (start 157.85 154.61) (end 160.71 151.75) (width 0.75) (layer F.Cu) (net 5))
 (segment (start 157.85 177.44) (end 157.85 154.61) (width 0.75) (layer F.Cu) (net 5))
 (segment (start 163.29 182.88) (end 157.85 177.44) (width 0.75) (layer F.Cu) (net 5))
 (segment (start 225.74 182.88) (end 163.29 182.88) (width 0.75) (layer F.Cu) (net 5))
 (segment (start 229.15 179.47) (end 225.74 182.88) (width 0.75) (layer F.Cu) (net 5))
 (segment (start 229.15 177.21) (end 229.15 179.47) (width 0.75) (layer F.Cu) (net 5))
 (segment (start 227.23 175.29) (end 229.15 177.21) (width 0.75) (layer F.Cu) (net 5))
 (segment (start 227.23 173.66) (end 227.23 175.29) (width 0.75) (layer F.Cu) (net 5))
 (segment (start 226.52 172.95) (end 227.23 173.66) (width 0.75) (layer F.Cu) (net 5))
 (segment (start 209.59 154.8) (end 208.89 154.8) (width 0.254) (layer B.Cu) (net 13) (status C00000))
 (segment (start 174.69 171.32) (end 171.82 174.19) (width 0.254) (layer B.Cu) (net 13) (status 800000))
 (segment (start 199.92 171.32) (end 174.69 171.32) (width 0.254) (layer B.Cu) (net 13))
 (segment (start 201.9 169.34) (end 199.92 171.32) (width 0.254) (layer B.Cu) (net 13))
 (segment (start 201.9 167.25) (end 201.9 169.34) (width 0.254) (layer B.Cu) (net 13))
 (segment (start 204.95 164.2) (end 201.9 167.25) (width 0.254) (layer B.Cu) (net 13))
 (segment (start 204.95 158.74) (end 204.95 164.2) (width 0.254) (layer B.Cu) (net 13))
 (segment (start 208.89 154.8) (end 204.95 158.74) (width 0.254) (layer B.Cu) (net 13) (status 400000))
 (segment (start 161.42 158.04) (end 163.74 158.04) (width 0.254) (layer F.Cu) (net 20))
 (segment (start 161.24 171.23) (end 164.2 174.19) (width 0.254) (layer F.Cu) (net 20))
 (segment (start 161.24 163.49) (end 161.24 171.23) (width 0.254) (layer F.Cu) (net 20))
 (segment (start 164.18 160.55) (end 161.24 163.49) (width 0.254) (layer F.Cu) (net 20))
 (segment (start 164.18 158.48) (end 164.18 160.55) (width 0.254) (layer F.Cu) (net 20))
 (segment (start 163.74 158.04) (end 164.18 158.48) (width 0.254) (layer F.Cu) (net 20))
 (segment (start 212.09 157.3) (end 213.76 157.3) (width 0.254) (layer B.Cu) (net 16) (status 400000))
 (segment (start 169.28 177.82) (end 169.28 174.19) (width 0.254) (layer B.Cu) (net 16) (status 800000))
 (segment (start 171.39 179.93) (end 169.28 177.82) (width 0.254) (layer B.Cu) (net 16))
 (segment (start 214.17 179.93) (end 171.39 179.93) (width 0.254) (layer B.Cu) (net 16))
 (segment (start 216.74 177.36) (end 214.17 179.93) (width 0.254) (layer B.Cu) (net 16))
 (segment (start 216.74 160.28) (end 216.74 177.36) (width 0.254) (layer B.Cu) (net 16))
 (segment (start 213.76 157.3) (end 216.74 160.28) (width 0.254) (layer B.Cu) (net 16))
 (segment (start 209.59 157.3) (end 207.76 157.3) (width 0.254) (layer B.Cu) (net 14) (status 400000))
 (segment (start 176.44 172.11) (end 174.36 174.19) (width 0.254) (layer B.Cu) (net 14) (status 800000))
 (segment (start 200.55 172.11) (end 176.44 172.11) (width 0.254) (layer B.Cu) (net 14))
 (segment (start 202.9 169.76) (end 200.55 172.11) (width 0.254) (layer B.Cu) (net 14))
 (segment (start 202.9 167.7) (end 202.9 169.76) (width 0.254) (layer B.Cu) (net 14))
 (segment (start 205.81 164.79) (end 202.9 167.7) (width 0.254) (layer B.Cu) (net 14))
 (segment (start 205.81 159.25) (end 205.81 164.79) (width 0.254) (layer B.Cu) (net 14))
 (segment (start 207.76 157.3) (end 205.81 159.25) (width 0.254) (layer B.Cu) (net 14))
 (segment (start 209.59 159.8) (end 207.43 159.8) (width 0.254) (layer F.Cu) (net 15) (status 400000))
 (segment (start 200.66 166.57) (end 197.22 166.57) (width 0.254) (layer F.Cu) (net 15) (status 800000))
 (segment (start 207.43 159.8) (end 200.66 166.57) (width 0.254) (layer F.Cu) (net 15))
 (segment (start 213 176.27) (end 213 177.2) (width 0.254) (layer F.Cu) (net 19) (status 400000))
 (segment (start 176.9 169.23) (end 176.9 166.57) (width 0.254) (layer F.Cu) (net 19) (status 800000))
 (segment (start 180.75 173.08) (end 176.9 169.23) (width 0.254) (layer F.Cu) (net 19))
 (segment (start 180.75 176.84) (end 180.75 173.08) (width 0.254) (layer F.Cu) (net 19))
 (segment (start 182.45 178.54) (end 180.75 176.84) (width 0.254) (layer F.Cu) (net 19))
 (segment (start 211.66 178.54) (end 182.45 178.54) (width 0.254) (layer F.Cu) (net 19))
 (segment (start 213 177.2) (end 211.66 178.54) (width 0.254) (layer F.Cu) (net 19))
 (segment (start 192.14 166.57) (end 191.98 166.57) (width 0.254) (layer F.Cu) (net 17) (status C00000))
 (segment (start 180.98 162.8) (end 179.27 161.09) (width 0.254) (layer F.Cu) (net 17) (status 800000))
 (segment (start 184.45 162.8) (end 180.98 162.8) (width 0.254) (layer F.Cu) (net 17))
 (segment (start 186.51 164.86) (end 184.45 162.8) (width 0.254) (layer F.Cu) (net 17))
 (segment (start 190.27 164.86) (end 186.51 164.86) (width 0.254) (layer F.Cu) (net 17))
 (segment (start 191.98 166.57) (end 190.27 164.86) (width 0.254) (layer F.Cu) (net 17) (status 400000))
 (segment (start 194.68 166.57) (end 194.61 166.57) (width 0.254) (layer F.Cu) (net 18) (status C00000))
 (segment (start 186.96 163.79) (end 184.33 161.16) (width 0.254) (layer F.Cu) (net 18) (status 800000))
 (segment (start 191.83 163.79) (end 186.96 163.79) (width 0.254) (layer F.Cu) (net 18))
 (segment (start 194.61 166.57) (end 191.83 163.79) (width 0.254) (layer F.Cu) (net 18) (status 400000)))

